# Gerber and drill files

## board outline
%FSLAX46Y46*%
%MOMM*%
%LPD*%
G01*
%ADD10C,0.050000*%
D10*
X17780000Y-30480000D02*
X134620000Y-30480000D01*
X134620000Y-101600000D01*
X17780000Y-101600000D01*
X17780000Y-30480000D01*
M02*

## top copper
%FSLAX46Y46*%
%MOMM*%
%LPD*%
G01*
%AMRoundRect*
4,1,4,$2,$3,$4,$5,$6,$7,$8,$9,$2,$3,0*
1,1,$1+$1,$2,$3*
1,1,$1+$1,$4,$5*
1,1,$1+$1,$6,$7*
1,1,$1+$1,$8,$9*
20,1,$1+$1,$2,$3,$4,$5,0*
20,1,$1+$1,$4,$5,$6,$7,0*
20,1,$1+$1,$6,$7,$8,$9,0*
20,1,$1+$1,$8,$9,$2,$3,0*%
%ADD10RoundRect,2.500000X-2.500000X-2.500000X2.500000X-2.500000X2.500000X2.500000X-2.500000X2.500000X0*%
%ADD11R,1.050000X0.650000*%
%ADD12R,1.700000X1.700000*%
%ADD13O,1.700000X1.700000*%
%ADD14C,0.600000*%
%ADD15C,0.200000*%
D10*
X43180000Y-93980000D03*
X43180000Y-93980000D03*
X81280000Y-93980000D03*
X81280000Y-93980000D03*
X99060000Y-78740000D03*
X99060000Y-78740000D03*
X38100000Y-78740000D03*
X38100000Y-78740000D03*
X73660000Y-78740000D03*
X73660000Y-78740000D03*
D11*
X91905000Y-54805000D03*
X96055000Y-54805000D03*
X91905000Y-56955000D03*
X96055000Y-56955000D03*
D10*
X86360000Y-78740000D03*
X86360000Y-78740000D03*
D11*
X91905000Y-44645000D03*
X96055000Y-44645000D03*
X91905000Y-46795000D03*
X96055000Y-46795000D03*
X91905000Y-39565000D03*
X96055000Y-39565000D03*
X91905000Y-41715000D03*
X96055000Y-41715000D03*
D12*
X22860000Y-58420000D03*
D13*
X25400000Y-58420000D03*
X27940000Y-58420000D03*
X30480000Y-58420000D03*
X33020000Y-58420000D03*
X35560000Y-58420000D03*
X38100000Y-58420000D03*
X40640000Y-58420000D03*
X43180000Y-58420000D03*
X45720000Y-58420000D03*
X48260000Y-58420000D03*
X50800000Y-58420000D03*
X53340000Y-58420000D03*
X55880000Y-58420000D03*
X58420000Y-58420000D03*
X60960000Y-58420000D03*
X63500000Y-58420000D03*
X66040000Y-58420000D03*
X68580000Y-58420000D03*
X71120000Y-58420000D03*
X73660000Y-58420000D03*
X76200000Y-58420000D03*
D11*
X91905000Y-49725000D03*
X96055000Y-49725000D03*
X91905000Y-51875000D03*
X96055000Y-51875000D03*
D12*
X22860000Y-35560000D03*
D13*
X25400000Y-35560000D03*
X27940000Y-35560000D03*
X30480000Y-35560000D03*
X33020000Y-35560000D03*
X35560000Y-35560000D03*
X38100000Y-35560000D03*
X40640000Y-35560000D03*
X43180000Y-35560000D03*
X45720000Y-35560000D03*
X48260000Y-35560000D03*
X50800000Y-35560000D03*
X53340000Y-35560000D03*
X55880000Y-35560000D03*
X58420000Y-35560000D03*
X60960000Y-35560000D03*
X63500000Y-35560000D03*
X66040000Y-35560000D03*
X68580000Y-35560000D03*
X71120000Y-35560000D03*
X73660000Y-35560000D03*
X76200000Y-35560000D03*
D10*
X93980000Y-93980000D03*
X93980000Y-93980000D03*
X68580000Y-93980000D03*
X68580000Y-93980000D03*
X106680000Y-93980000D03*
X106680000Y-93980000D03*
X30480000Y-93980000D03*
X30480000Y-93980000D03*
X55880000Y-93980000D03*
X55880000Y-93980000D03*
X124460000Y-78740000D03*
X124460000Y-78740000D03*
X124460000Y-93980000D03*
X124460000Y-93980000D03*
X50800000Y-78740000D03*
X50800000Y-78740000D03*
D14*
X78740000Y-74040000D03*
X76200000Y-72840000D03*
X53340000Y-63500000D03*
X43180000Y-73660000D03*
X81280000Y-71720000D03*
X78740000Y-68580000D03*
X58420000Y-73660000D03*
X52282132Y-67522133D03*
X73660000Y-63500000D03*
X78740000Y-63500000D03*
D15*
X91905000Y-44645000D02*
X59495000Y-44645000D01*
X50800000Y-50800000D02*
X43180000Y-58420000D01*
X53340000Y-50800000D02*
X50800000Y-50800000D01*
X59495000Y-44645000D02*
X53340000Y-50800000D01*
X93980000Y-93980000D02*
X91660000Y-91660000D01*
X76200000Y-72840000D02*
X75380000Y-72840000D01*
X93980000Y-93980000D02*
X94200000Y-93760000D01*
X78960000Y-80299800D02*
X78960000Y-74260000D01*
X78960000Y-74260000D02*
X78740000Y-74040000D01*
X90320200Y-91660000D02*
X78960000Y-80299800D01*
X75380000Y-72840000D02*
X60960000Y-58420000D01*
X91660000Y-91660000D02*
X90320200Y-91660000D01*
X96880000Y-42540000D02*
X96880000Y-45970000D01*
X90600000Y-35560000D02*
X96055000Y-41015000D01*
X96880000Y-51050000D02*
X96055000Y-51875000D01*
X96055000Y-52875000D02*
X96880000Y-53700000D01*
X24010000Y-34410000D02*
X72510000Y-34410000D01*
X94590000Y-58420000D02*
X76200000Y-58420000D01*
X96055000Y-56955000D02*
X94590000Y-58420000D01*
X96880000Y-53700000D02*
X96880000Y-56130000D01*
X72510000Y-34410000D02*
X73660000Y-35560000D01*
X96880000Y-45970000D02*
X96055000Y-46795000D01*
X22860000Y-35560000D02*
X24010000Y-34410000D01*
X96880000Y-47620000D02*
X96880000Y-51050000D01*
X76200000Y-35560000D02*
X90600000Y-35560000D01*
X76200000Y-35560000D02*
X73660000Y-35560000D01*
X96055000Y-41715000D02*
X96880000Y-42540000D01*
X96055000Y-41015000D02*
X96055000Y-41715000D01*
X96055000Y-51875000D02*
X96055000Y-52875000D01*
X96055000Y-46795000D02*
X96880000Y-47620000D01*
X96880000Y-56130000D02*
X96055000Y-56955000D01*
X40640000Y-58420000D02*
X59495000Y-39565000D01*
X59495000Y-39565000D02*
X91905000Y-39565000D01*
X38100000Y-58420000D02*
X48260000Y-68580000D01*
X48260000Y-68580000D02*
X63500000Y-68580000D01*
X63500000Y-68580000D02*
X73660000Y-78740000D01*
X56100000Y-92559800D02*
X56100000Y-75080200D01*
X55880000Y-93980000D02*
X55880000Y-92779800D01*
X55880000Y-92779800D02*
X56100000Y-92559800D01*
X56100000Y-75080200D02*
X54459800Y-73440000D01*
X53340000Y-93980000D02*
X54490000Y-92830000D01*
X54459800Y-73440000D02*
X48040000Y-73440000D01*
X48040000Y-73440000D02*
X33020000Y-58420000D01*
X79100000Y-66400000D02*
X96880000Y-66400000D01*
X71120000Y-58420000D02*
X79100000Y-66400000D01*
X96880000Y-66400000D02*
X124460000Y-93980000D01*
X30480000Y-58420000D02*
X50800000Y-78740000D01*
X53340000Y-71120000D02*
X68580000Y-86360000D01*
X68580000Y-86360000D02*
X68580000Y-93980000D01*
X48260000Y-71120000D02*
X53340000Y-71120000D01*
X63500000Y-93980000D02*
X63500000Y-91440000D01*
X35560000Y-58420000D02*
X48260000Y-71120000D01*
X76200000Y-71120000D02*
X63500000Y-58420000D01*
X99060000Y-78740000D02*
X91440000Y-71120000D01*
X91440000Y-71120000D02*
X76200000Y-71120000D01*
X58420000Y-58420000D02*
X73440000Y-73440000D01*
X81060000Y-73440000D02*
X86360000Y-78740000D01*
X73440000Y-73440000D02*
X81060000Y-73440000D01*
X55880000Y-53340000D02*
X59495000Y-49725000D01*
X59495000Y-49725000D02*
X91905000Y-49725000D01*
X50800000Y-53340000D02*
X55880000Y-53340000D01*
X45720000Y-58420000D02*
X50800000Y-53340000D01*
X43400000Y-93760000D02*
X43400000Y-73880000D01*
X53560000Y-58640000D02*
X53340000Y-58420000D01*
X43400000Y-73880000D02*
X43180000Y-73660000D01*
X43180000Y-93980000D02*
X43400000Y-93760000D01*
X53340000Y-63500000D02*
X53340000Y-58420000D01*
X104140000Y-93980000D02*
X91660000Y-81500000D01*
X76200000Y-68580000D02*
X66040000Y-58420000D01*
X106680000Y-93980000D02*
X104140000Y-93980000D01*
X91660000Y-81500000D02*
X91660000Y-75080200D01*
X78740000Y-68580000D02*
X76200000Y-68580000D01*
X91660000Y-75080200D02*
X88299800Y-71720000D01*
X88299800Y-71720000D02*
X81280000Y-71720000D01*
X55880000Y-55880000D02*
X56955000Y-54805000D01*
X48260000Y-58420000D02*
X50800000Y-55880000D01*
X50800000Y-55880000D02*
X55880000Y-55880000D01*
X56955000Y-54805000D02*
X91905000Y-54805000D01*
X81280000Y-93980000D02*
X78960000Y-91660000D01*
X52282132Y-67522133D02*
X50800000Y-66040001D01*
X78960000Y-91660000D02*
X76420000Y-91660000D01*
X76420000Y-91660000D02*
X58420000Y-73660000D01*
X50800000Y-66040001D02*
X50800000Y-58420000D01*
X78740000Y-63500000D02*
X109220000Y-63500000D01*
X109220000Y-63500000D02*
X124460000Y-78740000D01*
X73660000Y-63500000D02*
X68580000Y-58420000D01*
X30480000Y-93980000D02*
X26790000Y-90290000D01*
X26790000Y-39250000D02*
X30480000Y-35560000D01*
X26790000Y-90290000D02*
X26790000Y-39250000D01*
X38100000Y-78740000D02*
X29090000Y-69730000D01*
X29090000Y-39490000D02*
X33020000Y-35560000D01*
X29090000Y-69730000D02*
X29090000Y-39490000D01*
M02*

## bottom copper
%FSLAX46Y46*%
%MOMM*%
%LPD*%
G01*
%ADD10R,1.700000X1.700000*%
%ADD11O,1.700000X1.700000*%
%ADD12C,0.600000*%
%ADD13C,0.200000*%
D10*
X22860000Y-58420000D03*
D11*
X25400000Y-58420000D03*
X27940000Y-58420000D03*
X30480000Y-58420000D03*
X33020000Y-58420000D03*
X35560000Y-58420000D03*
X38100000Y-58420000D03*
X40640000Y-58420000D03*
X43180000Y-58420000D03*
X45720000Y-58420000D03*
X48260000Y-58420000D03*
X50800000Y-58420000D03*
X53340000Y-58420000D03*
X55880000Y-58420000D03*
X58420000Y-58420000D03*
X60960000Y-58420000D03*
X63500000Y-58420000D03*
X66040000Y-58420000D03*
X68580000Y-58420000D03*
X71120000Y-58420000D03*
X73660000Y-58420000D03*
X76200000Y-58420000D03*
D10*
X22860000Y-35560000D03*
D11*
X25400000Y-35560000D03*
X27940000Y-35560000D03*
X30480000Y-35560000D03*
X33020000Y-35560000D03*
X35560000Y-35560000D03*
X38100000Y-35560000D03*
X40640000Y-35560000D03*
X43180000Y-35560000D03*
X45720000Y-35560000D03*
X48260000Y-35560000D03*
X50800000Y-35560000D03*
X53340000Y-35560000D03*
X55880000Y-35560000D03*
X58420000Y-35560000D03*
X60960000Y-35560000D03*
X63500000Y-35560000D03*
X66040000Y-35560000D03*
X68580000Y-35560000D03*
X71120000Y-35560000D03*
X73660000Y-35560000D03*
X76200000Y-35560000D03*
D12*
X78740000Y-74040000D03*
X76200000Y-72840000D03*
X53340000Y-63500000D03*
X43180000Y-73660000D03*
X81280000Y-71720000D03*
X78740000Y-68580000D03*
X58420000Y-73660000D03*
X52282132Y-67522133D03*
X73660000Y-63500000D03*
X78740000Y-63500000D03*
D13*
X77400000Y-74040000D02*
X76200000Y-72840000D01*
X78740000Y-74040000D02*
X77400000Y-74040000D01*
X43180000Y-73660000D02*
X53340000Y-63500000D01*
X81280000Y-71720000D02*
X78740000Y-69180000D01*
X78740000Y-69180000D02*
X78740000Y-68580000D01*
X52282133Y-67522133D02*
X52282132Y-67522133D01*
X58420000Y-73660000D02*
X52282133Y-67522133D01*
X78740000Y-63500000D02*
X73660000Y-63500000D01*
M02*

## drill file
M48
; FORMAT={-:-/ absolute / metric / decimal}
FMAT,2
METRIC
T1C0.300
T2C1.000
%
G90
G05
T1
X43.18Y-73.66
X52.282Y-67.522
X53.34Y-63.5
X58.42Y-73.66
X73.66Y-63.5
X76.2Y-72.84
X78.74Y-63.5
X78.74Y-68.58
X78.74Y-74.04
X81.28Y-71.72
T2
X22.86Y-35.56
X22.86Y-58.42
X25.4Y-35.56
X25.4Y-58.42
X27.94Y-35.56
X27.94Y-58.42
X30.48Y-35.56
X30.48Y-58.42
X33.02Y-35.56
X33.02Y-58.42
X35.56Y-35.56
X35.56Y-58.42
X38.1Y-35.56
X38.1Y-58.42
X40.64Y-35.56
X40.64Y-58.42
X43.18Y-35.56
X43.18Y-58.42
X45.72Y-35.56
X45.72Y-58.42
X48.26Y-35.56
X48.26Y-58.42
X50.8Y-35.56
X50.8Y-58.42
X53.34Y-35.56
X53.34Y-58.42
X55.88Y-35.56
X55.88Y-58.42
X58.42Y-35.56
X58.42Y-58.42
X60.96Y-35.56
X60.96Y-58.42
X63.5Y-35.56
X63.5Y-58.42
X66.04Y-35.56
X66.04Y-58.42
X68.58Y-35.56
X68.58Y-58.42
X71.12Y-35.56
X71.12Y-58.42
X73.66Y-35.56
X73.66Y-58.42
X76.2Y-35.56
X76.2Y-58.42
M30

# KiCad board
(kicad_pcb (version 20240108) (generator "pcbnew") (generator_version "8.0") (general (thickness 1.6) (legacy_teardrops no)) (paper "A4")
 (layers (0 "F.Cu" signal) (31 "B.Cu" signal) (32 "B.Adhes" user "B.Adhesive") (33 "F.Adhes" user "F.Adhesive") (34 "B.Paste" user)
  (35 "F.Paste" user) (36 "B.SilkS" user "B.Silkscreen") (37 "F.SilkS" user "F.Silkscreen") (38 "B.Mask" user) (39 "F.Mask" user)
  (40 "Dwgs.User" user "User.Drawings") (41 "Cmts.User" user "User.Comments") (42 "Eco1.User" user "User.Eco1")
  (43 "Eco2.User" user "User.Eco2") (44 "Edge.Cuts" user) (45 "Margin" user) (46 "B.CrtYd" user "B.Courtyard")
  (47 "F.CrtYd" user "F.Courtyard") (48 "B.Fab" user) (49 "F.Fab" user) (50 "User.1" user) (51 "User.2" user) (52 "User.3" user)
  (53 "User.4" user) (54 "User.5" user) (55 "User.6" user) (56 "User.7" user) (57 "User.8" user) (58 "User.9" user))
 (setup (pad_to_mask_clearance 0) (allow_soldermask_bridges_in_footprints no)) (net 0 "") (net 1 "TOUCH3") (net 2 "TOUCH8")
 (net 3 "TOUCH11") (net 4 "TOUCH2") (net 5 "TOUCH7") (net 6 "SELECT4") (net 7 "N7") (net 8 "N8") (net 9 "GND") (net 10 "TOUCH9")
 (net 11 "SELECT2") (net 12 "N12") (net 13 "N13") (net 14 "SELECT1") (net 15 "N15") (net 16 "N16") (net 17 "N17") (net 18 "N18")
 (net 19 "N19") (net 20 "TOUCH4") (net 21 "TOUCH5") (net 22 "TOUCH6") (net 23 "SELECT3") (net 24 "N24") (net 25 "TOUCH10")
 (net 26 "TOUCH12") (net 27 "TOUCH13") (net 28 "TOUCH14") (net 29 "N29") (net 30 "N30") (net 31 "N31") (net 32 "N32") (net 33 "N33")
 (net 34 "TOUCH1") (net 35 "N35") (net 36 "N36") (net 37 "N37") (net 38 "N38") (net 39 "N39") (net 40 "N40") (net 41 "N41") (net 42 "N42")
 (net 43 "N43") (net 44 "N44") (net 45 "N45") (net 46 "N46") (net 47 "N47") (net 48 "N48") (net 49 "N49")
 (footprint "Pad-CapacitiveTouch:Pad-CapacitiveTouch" (layer "F.Cu") (at 43.18 93.98)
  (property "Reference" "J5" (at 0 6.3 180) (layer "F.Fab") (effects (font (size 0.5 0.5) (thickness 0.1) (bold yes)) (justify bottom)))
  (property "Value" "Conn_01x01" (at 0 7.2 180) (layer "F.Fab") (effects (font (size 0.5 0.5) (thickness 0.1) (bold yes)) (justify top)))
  (pad "1" smd roundrect (at 0 0) (size 10 10) (layers "F.Cu") (roundrect_rratio 0.25) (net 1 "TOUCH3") (thermal_bridge_angle 0))
  (pad "1" smd roundrect (at 0 0) (size 10 10) (layers "F.Cu" "F.Mask") (roundrect_rratio 0.25) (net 1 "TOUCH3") (thermal_bridge_angle 0)))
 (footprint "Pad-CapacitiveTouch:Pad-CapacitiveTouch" (layer "F.Cu") (at 81.28 93.98)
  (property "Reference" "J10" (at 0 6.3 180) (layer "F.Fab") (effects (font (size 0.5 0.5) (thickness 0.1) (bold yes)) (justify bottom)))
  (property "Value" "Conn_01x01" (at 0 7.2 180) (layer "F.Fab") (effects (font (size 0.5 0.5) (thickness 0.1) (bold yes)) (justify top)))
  (pad "1" smd roundrect (at 0 0) (size 10 10) (layers "F.Cu") (roundrect_rratio 0.25) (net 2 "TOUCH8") (thermal_bridge_angle 0))
  (pad "1" smd roundrect (at 0 0) (size 10 10) (layers "F.Cu" "F.Mask") (roundrect_rratio 0.25) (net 2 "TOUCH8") (thermal_bridge_angle 0)))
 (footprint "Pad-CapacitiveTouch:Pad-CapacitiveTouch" (layer "F.Cu") (at 99.06 78.74)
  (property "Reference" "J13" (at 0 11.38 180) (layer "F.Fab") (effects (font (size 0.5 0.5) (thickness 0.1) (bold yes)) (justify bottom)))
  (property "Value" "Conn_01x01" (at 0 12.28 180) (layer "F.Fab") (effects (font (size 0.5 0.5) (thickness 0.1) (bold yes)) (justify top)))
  (pad "1" smd roundrect (at 0 0) (size 10 10) (layers "F.Cu") (roundrect_rratio 0.25) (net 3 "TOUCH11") (thermal_bridge_angle 0))
  (pad "1" smd roundrect (at 0 0) (size 10 10) (layers "F.Cu" "F.Mask") (roundrect_rratio 0.25) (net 3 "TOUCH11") (thermal_bridge_angle 0)))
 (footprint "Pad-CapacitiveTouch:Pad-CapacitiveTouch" (layer "F.Cu") (at 38.1 78.74)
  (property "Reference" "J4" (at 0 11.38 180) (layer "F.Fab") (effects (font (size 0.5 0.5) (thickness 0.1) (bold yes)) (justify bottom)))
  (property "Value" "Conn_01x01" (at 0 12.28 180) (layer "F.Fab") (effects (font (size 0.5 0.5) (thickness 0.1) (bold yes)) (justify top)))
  (pad "1" smd roundrect (at 0 0) (size 10 10) (layers "F.Cu") (roundrect_rratio 0.25) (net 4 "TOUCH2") (thermal_bridge_angle 0))
  (pad "1" smd roundrect (at 0 0) (size 10 10) (layers "F.Cu" "F.Mask") (roundrect_rratio 0.25) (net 4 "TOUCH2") (thermal_bridge_angle 0)))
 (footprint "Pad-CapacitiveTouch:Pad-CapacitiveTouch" (layer "F.Cu") (at 73.66 78.74)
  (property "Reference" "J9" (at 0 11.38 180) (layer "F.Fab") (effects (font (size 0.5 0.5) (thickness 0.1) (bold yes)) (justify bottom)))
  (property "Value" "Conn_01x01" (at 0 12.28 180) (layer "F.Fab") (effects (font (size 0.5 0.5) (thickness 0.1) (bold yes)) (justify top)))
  (pad "1" smd roundrect (at 0 0) (size 10 10) (layers "F.Cu") (roundrect_rratio 0.25) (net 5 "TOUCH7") (thermal_bridge_angle 0))
  (pad "1" smd roundrect (at 0 0) (size 10 10) (layers "F.Cu" "F.Mask") (roundrect_rratio 0.25) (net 5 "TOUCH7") (thermal_bridge_angle 0)))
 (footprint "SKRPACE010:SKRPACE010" (layer "F.Cu") (at 93.98 55.88)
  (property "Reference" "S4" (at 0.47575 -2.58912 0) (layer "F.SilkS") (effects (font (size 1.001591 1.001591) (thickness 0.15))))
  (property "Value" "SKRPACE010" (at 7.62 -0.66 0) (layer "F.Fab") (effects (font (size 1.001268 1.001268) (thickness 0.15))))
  (pad "1" smd rect (at -2.075 -1.075) (size 1.05 0.65) (layers "F.Cu" "F.Paste" "F.Mask") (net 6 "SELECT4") (solder_mask_margin 0.102))
  (pad "2" smd rect (at 2.075 -1.075) (size 1.05 0.65) (layers "F.Cu" "F.Paste" "F.Mask") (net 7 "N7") (solder_mask_margin 0.102))
  (pad "3" smd rect (at -2.075 1.075) (size 1.05 0.65) (layers "F.Cu" "F.Paste" "F.Mask") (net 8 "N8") (solder_mask_margin 0.102))
  (pad "4" smd rect (at 2.075 1.075) (size 1.05 0.65) (layers "F.Cu" "F.Paste" "F.Mask") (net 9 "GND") (solder_mask_margin 0.102)))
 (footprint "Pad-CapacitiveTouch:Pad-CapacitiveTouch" (layer "F.Cu") (at 86.36 78.74)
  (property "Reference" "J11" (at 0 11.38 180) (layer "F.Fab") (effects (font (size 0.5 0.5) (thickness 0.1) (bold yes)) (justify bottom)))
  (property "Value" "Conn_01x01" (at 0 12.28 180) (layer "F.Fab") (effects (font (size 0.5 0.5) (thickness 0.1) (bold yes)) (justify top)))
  (pad "1" smd roundrect (at 0 0) (size 10 10) (layers "F.Cu") (roundrect_rratio 0.25) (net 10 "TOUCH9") (thermal_bridge_angle 0))
  (pad "1" smd roundrect (at 0 0) (size 10 10) (layers "F.Cu" "F.Mask") (roundrect_rratio 0.25) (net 10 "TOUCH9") (thermal_bridge_angle 0)))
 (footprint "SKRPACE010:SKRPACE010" (layer "F.Cu") (at 93.98 45.72)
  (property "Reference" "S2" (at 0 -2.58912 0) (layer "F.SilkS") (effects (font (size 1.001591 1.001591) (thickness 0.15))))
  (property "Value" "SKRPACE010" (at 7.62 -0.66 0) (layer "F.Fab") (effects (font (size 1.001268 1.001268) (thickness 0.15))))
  (pad "1" smd rect (at -2.075 -1.075) (size 1.05 0.65) (layers "F.Cu" "F.Paste" "F.Mask") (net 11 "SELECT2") (solder_mask_margin 0.102))
  (pad "2" smd rect (at 2.075 -1.075) (size 1.05 0.65) (layers "F.Cu" "F.Paste" "F.Mask") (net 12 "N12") (solder_mask_margin 0.102))
  (pad "3" smd rect (at -2.075 1.075) (size 1.05 0.65) (layers "F.Cu" "F.Paste" "F.Mask") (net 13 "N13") (solder_mask_margin 0.102))
  (pad "4" smd rect (at 2.075 1.075) (size 1.05 0.65) (layers "F.Cu" "F.Paste" "F.Mask") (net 9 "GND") (solder_mask_margin 0.102)))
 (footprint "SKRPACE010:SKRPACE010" (layer "F.Cu") (at 93.98 40.64)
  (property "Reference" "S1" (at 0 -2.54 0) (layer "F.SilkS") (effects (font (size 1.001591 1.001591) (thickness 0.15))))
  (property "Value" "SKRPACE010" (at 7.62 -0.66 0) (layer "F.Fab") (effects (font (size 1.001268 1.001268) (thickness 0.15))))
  (pad "1" smd rect (at -2.075 -1.075) (size 1.05 0.65) (layers "F.Cu" "F.Paste" "F.Mask") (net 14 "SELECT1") (solder_mask_margin 0.102))
  (pad "2" smd rect (at 2.075 -1.075) (size 1.05 0.65) (layers "F.Cu" "F.Paste" "F.Mask") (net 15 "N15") (solder_mask_margin 0.102))
  (pad "3" smd rect (at -2.075 1.075) (size 1.05 0.65) (layers "F.Cu" "F.Paste" "F.Mask") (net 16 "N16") (solder_mask_margin 0.102))
  (pad "4" smd rect (at 2.075 1.075) (size 1.05 0.65) (layers "F.Cu" "F.Paste" "F.Mask") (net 9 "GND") (solder_mask_margin 0.102)))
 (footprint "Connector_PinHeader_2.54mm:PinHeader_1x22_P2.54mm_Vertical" (layer "F.Cu") (at 22.86 58.42 90)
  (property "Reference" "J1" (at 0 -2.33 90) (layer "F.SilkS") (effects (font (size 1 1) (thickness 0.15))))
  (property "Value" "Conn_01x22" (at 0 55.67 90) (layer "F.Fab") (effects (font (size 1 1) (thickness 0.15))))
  (pad "1" thru_hole rect (at 0 0 90) (size 1.7 1.7) (drill 1) (layers "*.Cu" "*.Mask") (remove_unused_layers no) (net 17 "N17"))
  (pad "2" thru_hole oval (at 0 2.54 90) (size 1.7 1.7) (drill 1) (layers "*.Cu" "*.Mask") (remove_unused_layers no) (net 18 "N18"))
  (pad "3" thru_hole oval (at 0 5.08 90) (size 1.7 1.7) (drill 1) (layers "*.Cu" "*.Mask") (remove_unused_layers no) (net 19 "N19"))
  (pad "4" thru_hole oval (at 0 7.62 90) (size 1.7 1.7) (drill 1) (layers "*.Cu" "*.Mask") (remove_unused_layers no) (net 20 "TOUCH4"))
  (pad "5" thru_hole oval (at 0 10.16 90) (size 1.7 1.7) (drill 1) (layers "*.Cu" "*.Mask") (remove_unused_layers no) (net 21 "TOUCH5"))
  (pad "6" thru_hole oval (at 0 12.7 90) (size 1.7 1.7) (drill 1) (layers "*.Cu" "*.Mask") (remove_unused_layers no) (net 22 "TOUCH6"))
  (pad "7" thru_hole oval (at 0 15.24 90) (size 1.7 1.7) (drill 1) (layers "*.Cu" "*.Mask") (remove_unused_layers no) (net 5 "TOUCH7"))
  (pad "8" thru_hole oval (at 0 17.78 90) (size 1.7 1.7) (drill 1) (layers "*.Cu" "*.Mask") (remove_unused_layers no) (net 14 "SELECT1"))
  (pad "9" thru_hole oval (at 0 20.32 90) (size 1.7 1.7) (drill 1) (layers "*.Cu" "*.Mask") (remove_unused_layers no) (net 11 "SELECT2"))
  (pad "10" thru_hole oval (at 0 22.86 90) (size 1.7 1.7) (drill 1) (layers "*.Cu" "*.Mask") (remove_unused_layers no) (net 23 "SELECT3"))
  (pad "11" thru_hole oval (at 0 25.4 90) (size 1.7 1.7) (drill 1) (layers "*.Cu" "*.Mask") (remove_unused_layers no) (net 6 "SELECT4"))
  (pad "12" thru_hole oval (at 0 27.94 90) (size 1.7 1.7) (drill 1) (layers "*.Cu" "*.Mask") (remove_unused_layers no) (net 2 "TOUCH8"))
  (pad "13" thru_hole oval (at 0 30.48 90) (size 1.7 1.7) (drill 1) (layers "*.Cu" "*.Mask") (remove_unused_layers no) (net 1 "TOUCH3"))
  (pad "14" thru_hole oval (at 0 33.02 90) (size 1.7 1.7) (drill 1) (layers "*.Cu" "*.Mask") (remove_unused_layers no) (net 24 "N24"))
  (pad "15" thru_hole oval (at 0 35.56 90) (size 1.7 1.7) (drill 1) (layers "*.Cu" "*.Mask") (remove_unused_layers no) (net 10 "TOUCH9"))
  (pad "16" thru_hole oval (at 0 38.1 90) (size 1.7 1.7) (drill 1) (layers "*.Cu" "*.Mask") (remove_unused_layers no) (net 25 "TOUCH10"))
  (pad "17" thru_hole oval (at 0 40.64 90) (size 1.7 1.7) (drill 1) (layers "*.Cu" "*.Mask") (remove_unused_layers no) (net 3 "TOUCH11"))
  (pad "18" thru_hole oval (at 0 43.18 90) (size 1.7 1.7) (drill 1) (layers "*.Cu" "*.Mask") (remove_unused_layers no) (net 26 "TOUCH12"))
  (pad "19" thru_hole oval (at 0 45.72 90) (size 1.7 1.7) (drill 1) (layers "*.Cu" "*.Mask") (remove_unused_layers no) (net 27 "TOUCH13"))
  (pad "20" thru_hole oval (at 0 48.26 90) (size 1.7 1.7) (drill 1) (layers "*.Cu" "*.Mask") (remove_unused_layers no) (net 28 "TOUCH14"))
  (pad "21" thru_hole oval (at 0 50.8 90) (size 1.7 1.7) (drill 1) (layers "*.Cu" "*.Mask") (remove_unused_layers no) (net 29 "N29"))
  (pad "22" thru_hole oval (at 0 53.34 90) (size 1.7 1.7) (drill 1) (layers "*.Cu" "*.Mask") (remove_unused_layers no) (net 9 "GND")))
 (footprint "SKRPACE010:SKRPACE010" (layer "F.Cu") (at 93.98 50.8)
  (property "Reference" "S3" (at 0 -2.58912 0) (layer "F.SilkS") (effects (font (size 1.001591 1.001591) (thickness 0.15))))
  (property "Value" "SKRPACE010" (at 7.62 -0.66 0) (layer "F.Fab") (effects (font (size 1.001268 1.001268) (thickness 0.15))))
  (pad "1" smd rect (at -2.075 -1.075) (size 1.05 0.65) (layers "F.Cu" "F.Paste" "F.Mask") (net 23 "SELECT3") (solder_mask_margin 0.102))
  (pad "2" smd rect (at 2.075 -1.075) (size 1.05 0.65) (layers "F.Cu" "F.Paste" "F.Mask") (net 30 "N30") (solder_mask_margin 0.102))
  (pad "3" smd rect (at -2.075 1.075) (size 1.05 0.65) (layers "F.Cu" "F.Paste" "F.Mask") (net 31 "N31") (solder_mask_margin 0.102))
  (pad "4" smd rect (at 2.075 1.075) (size 1.05 0.65) (layers "F.Cu" "F.Paste" "F.Mask") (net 9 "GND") (solder_mask_margin 0.102)))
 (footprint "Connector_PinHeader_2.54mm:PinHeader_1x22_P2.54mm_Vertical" (layer "F.Cu") (at 22.86 35.56 90)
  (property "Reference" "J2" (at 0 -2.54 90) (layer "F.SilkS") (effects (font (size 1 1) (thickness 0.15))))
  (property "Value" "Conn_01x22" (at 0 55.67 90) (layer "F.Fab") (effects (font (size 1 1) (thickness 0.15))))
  (pad "1" thru_hole rect (at 0 0 90) (size 1.7 1.7) (drill 1) (layers "*.Cu" "*.Mask") (remove_unused_layers no) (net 9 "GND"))
  (pad "2" thru_hole oval (at 0 2.54 90) (size 1.7 1.7) (drill 1) (layers "*.Cu" "*.Mask") (remove_unused_layers no) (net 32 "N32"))
  (pad "3" thru_hole oval (at 0 5.08 90) (size 1.7 1.7) (drill 1) (layers "*.Cu" "*.Mask") (remove_unused_layers no) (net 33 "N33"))
  (pad "4" thru_hole oval (at 0 7.62 90) (size 1.7 1.7) (drill 1) (layers "*.Cu" "*.Mask") (remove_unused_layers no) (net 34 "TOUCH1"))
  (pad "5" thru_hole oval (at 0 10.16 90) (size 1.7 1.7) (drill 1) (layers "*.Cu" "*.Mask") (remove_unused_layers no) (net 4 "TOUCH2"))
  (pad "6" thru_hole oval (at 0 12.7 90) (size 1.7 1.7) (drill 1) (layers "*.Cu" "*.Mask") (remove_unused_layers no) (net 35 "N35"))
  (pad "7" thru_hole oval (at 0 15.24 90) (size 1.7 1.7) (drill 1) (layers "*.Cu" "*.Mask") (remove_unused_layers no) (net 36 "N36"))
  (pad "8" thru_hole oval (at 0 17.78 90) (size 1.7 1.7) (drill 1) (layers "*.Cu" "*.Mask") (remove_unused_layers no) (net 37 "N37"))
  (pad "9" thru_hole oval (at 0 20.32 90) (size 1.7 1.7) (drill 1) (layers "*.Cu" "*.Mask") (remove_unused_layers no) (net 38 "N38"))
  (pad "10" thru_hole oval (at 0 22.86 90) (size 1.7 1.7) (drill 1) (layers "*.Cu" "*.Mask") (remove_unused_layers no) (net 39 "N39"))
  (pad "11" thru_hole oval (at 0 25.4 90) (size 1.7 1.7) (drill 1) (layers "*.Cu" "*.Mask") (remove_unused_layers no) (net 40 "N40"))
  (pad "12" thru_hole oval (at 0 27.94 90) (size 1.7 1.7) (drill 1) (layers "*.Cu" "*.Mask") (remove_unused_layers no) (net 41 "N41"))
  (pad "13" thru_hole oval (at 0 30.48 90) (size 1.7 1.7) (drill 1) (layers "*.Cu" "*.Mask") (remove_unused_layers no) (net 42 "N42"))
  (pad "14" thru_hole oval (at 0 33.02 90) (size 1.7 1.7) (drill 1) (layers "*.Cu" "*.Mask") (remove_unused_layers no) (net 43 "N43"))
  (pad "15" thru_hole oval (at 0 35.56 90) (size 1.7 1.7) (drill 1) (layers "*.Cu" "*.Mask") (remove_unused_layers no) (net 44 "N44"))
  (pad "16" thru_hole oval (at 0 38.1 90) (size 1.7 1.7) (drill 1) (layers "*.Cu" "*.Mask") (remove_unused_layers no) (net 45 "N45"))
  (pad "17" thru_hole oval (at 0 40.64 90) (size 1.7 1.7) (drill 1) (layers "*.Cu" "*.Mask") (remove_unused_layers no) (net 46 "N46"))
  (pad "18" thru_hole oval (at 0 43.18 90) (size 1.7 1.7) (drill 1) (layers "*.Cu" "*.Mask") (remove_unused_layers no) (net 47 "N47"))
  (pad "19" thru_hole oval (at 0 45.72 90) (size 1.7 1.7) (drill 1) (layers "*.Cu" "*.Mask") (remove_unused_layers no) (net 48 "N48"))
  (pad "20" thru_hole oval (at 0 48.26 90) (size 1.7 1.7) (drill 1) (layers "*.Cu" "*.Mask") (remove_unused_layers no) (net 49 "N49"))
  (pad "21" thru_hole oval (at 0 50.8 90) (size 1.7 1.7) (drill 1) (layers "*.Cu" "*.Mask") (remove_unused_layers no) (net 9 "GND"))
  (pad "22" thru_hole oval (at 0 53.34 90) (size 1.7 1.7) (drill 1) (layers "*.Cu" "*.Mask") (remove_unused_layers no) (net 9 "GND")))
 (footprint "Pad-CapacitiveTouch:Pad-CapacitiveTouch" (layer "F.Cu") (at 93.98 93.98)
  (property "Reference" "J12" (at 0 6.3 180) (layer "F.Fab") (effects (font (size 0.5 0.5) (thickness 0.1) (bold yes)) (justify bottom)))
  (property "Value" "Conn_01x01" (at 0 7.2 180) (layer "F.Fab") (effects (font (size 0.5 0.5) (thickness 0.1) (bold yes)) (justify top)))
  (pad "1" smd roundrect (at 0 0) (size 10 10) (layers "F.Cu") (roundrect_rratio 0.25) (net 25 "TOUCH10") (thermal_bridge_angle 0))
  (pad "1" smd roundrect (at 0 0) (size 10 10) (layers "F.Cu" "F.Mask") (roundrect_rratio 0.25) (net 25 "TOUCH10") (thermal_bridge_angle 0)))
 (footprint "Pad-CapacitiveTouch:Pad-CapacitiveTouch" (layer "F.Cu") (at 68.58 93.98)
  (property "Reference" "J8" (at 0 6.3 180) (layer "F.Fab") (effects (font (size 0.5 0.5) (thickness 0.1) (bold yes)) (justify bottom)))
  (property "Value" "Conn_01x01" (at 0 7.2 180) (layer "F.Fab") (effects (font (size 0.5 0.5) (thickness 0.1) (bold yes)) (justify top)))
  (pad "1" smd roundrect (at 0 0) (size 10 10) (layers "F.Cu") (roundrect_rratio 0.25) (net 22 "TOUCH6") (thermal_bridge_angle 0))
  (pad "1" smd roundrect (at 0 0) (size 10 10) (layers "F.Cu" "F.Mask") (roundrect_rratio 0.25) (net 22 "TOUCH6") (thermal_bridge_angle 0)))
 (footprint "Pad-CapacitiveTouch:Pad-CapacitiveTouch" (layer "F.Cu") (at 106.68 93.98)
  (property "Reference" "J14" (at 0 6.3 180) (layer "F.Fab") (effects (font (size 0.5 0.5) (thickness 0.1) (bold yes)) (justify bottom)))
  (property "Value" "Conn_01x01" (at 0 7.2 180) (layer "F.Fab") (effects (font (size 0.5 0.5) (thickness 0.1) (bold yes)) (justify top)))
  (pad "1" smd roundrect (at 0 0) (size 10 10) (layers "F.Cu") (roundrect_rratio 0.25) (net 26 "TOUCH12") (thermal_bridge_angle 0))
  (pad "1" smd roundrect (at 0 0) (size 10 10) (layers "F.Cu" "F.Mask") (roundrect_rratio 0.25) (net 26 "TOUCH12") (thermal_bridge_angle 0)))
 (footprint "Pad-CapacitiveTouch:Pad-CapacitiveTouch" (layer "F.Cu") (at 30.48 93.98)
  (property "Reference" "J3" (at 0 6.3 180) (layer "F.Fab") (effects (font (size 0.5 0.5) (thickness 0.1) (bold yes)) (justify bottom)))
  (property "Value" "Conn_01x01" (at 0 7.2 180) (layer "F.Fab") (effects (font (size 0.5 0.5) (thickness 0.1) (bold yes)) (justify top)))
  (pad "1" smd roundrect (at 0 0) (size 10 10) (layers "F.Cu") (roundrect_rratio 0.25) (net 34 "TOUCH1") (thermal_bridge_angle 0))
  (pad "1" smd roundrect (at 0 0) (size 10 10) (layers "F.Cu" "F.Mask") (roundrect_rratio 0.25) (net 34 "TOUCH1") (thermal_bridge_angle 0)))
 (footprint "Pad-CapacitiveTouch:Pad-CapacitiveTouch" (layer "F.Cu") (at 55.88 93.98)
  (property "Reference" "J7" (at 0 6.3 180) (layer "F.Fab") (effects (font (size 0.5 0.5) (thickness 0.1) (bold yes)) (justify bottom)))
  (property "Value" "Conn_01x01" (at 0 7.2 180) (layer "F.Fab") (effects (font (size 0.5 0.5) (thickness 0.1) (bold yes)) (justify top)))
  (pad "1" smd roundrect (at 0 0) (size 10 10) (layers "F.Cu") (roundrect_rratio 0.25) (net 21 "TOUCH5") (thermal_bridge_angle 0))
  (pad "1" smd roundrect (at 0 0) (size 10 10) (layers "F.Cu" "F.Mask") (roundrect_rratio 0.25) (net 21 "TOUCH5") (thermal_bridge_angle 0)))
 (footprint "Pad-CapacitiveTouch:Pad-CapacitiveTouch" (layer "F.Cu") (at 124.46 78.74)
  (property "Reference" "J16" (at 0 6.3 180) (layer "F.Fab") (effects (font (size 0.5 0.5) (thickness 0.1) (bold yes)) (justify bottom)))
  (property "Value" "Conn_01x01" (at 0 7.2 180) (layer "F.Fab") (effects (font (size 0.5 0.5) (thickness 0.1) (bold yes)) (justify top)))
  (pad "1" smd roundrect (at 0 0) (size 10 10) (layers "F.Cu") (roundrect_rratio 0.25) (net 27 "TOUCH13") (thermal_bridge_angle 0))
  (pad "1" smd roundrect (at 0 0) (size 10 10) (layers "F.Cu" "F.Mask") (roundrect_rratio 0.25) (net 27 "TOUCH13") (thermal_bridge_angle 0)))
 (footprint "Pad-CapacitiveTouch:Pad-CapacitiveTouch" (layer "F.Cu") (at 124.46 93.98)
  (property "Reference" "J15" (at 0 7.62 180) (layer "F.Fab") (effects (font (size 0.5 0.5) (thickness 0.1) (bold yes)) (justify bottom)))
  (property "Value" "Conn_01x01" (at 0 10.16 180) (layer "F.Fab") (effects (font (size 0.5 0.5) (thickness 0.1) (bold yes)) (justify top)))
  (pad "1" smd roundrect (at 0 0) (size 10 10) (layers "F.Cu") (roundrect_rratio 0.25) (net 28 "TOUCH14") (thermal_bridge_angle 0))
  (pad "1" smd roundrect (at 0 0) (size 10 10) (layers "F.Cu" "F.Mask") (roundrect_rratio 0.25) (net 28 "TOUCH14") (thermal_bridge_angle 0)))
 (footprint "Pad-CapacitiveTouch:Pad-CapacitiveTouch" (layer "F.Cu") (at 50.8 78.74)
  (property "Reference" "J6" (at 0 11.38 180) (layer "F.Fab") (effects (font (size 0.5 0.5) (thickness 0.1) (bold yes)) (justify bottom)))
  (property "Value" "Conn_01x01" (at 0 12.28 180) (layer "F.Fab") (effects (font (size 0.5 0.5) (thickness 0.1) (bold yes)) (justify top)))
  (pad "1" smd roundrect (at 0 0) (size 10 10) (layers "F.Cu") (roundrect_rratio 0.25) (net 20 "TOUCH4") (thermal_bridge_angle 0))
  (pad "1" smd roundrect (at 0 0) (size 10 10) (layers "F.Cu" "F.Mask") (roundrect_rratio 0.25) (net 20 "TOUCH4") (thermal_bridge_angle 0)))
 (gr_rect (start 17.78 30.48) (end 134.62 101.6) (stroke (width 0.05) (type default)) (fill none) (layer "Edge.Cuts"))
 (segment (start 91.905 44.645) (end 59.495 44.645) (width 0.2) (layer "F.Cu") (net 11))
 (segment (start 50.8 50.8) (end 43.18 58.42) (width 0.2) (layer "F.Cu") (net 11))
 (segment (start 53.34 50.8) (end 50.8 50.8) (width 0.2) (layer "F.Cu") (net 11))
 (segment (start 59.495 44.645) (end 53.34 50.8) (width 0.2) (layer "F.Cu") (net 11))
 (segment (start 93.98 93.98) (end 91.66 91.66) (width 0.2) (layer "F.Cu") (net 25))
 (segment (start 76.2 72.84) (end 75.38 72.84) (width 0.2) (layer "F.Cu") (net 25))
 (segment (start 93.98 93.98) (end 94.2 93.76) (width 0.2) (layer "F.Cu") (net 25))
 (segment (start 78.96 80.2998) (end 78.96 74.26) (width 0.2) (layer "F.Cu") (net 25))
 (segment (start 78.96 74.26) (end 78.74 74.04) (width 0.2) (layer "F.Cu") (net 25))
 (segment (start 90.3202 91.66) (end 78.96 80.2998) (width 0.2) (layer "F.Cu") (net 25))
 (segment (start 75.38 72.84) (end 60.96 58.42) (width 0.2) (layer "F.Cu") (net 25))
 (segment (start 91.66 91.66) (end 90.3202 91.66) (width 0.2) (layer "F.Cu") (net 25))
 (via (at 78.74 74.04) (size 0.6) (drill 0.3) (layers "F.Cu" "B.Cu") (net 25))
 (via (at 76.2 72.84) (size 0.6) (drill 0.3) (layers "F.Cu" "B.Cu") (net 25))
 (segment (start 77.4 74.04) (end 76.2 72.84) (width 0.2) (layer "B.Cu") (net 25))
 (segment (start 78.74 74.04) (end 77.4 74.04) (width 0.2) (layer "B.Cu") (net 25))
 (segment (start 96.88 42.54) (end 96.88 45.97) (width 0.2) (layer "F.Cu") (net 9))
 (segment (start 90.6 35.56) (end 96.055 41.015) (width 0.2) (layer "F.Cu") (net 9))
 (segment (start 96.88 51.05) (end 96.055 51.875) (width 0.2) (layer "F.Cu") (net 9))
 (segment (start 96.055 52.875) (end 96.88 53.7) (width 0.2) (layer "F.Cu") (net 9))
 (segment (start 24.01 34.41) (end 72.51 34.41) (width 0.2) (layer "F.Cu") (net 9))
 (segment (start 94.59 58.42) (end 76.2 58.42) (width 0.2) (layer "F.Cu") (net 9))
 (segment (start 96.055 56.955) (end 94.59 58.42) (width 0.2) (layer "F.Cu") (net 9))
 (segment (start 96.88 53.7) (end 96.88 56.13) (width 0.2) (layer "F.Cu") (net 9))
 (segment (start 72.51 34.41) (end 73.66 35.56) (width 0.2) (layer "F.Cu") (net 9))
 (segment (start 96.88 45.97) (end 96.055 46.795) (width 0.2) (layer "F.Cu") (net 9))
 (segment (start 22.86 35.56) (end 24.01 34.41) (width 0.2) (layer "F.Cu") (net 9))
 (segment (start 96.88 47.62) (end 96.88 51.05) (width 0.2) (layer "F.Cu") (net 9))
 (segment (start 76.2 35.56) (end 90.6 35.56) (width 0.2) (layer "F.Cu") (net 9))
 (segment (start 76.2 35.56) (end 73.66 35.56) (width 0.2) (layer "F.Cu") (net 9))
 (segment (start 96.055 41.715) (end 96.88 42.54) (width 0.2) (layer "F.Cu") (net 9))
 (segment (start 96.055 41.015) (end 96.055 41.715) (width 0.2) (layer "F.Cu") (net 9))
 (segment (start 96.055 51.875) (end 96.055 52.875) (width 0.2) (layer "F.Cu") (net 9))
 (segment (start 96.055 46.795) (end 96.88 47.62) (width 0.2) (layer "F.Cu") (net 9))
 (segment (start 96.88 56.13) (end 96.055 56.955) (width 0.2) (layer "F.Cu") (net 9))
 (segment (start 40.64 58.42) (end 59.495 39.565) (width 0.2) (layer "F.Cu") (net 14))
 (segment (start 59.495 39.565) (end 91.905 39.565) (width 0.2) (layer "F.Cu") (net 14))
 (segment (start 38.1 58.42) (end 48.26 68.58) (width 0.2) (layer "F.Cu") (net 5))
 (segment (start 48.26 68.58) (end 63.5 68.58) (width 0.2) (layer "F.Cu") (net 5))
 (segment (start 63.5 68.58) (end 73.66 78.74) (width 0.2) (layer "F.Cu") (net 5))
 (segment (start 56.1 92.5598) (end 56.1 75.0802) (width 0.2) (layer "F.Cu") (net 21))
 (segment (start 55.88 93.98) (end 55.88 92.7798) (width 0.2) (layer "F.Cu") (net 21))
 (segment (start 55.88 92.7798) (end 56.1 92.5598) (width 0.2) (layer "F.Cu") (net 21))
 (segment (start 56.1 75.0802) (end 54.4598 73.44) (width 0.2) (layer "F.Cu") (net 21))
 (segment (start 53.34 93.98) (end 54.49 92.83) (width 0.2) (layer "F.Cu") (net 21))
 (segment (start 54.4598 73.44) (end 48.04 73.44) (width 0.2) (layer "F.Cu") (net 21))
 (segment (start 48.04 73.44) (end 33.02 58.42) (width 0.2) (layer "F.Cu") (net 21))
 (segment (start 79.1 66.4) (end 96.88 66.4) (width 0.2) (layer "F.Cu") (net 28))
 (segment (start 71.12 58.42) (end 79.1 66.4) (width 0.2) (layer "F.Cu") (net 28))
 (segment (start 96.88 66.4) (end 124.46 93.98) (width 0.2) (layer "F.Cu") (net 28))
 (segment (start 30.48 58.42) (end 50.8 78.74) (width 0.2) (layer "F.Cu") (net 20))
 (segment (start 53.34 71.12) (end 68.58 86.36) (width 0.2) (layer "F.Cu") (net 22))
 (segment (start 68.58 86.36) (end 68.58 93.98) (width 0.2) (layer "F.Cu") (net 22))
 (segment (start 48.26 71.12) (end 53.34 71.12) (width 0.2) (layer "F.Cu") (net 22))
 (segment (start 63.5 93.98) (end 63.5 91.44) (width 0.2) (layer "F.Cu") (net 22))
 (segment (start 35.56 58.42) (end 48.26 71.12) (width 0.2) (layer "F.Cu") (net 22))
 (segment (start 76.2 71.12) (end 63.5 58.42) (width 0.2) (layer "F.Cu") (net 3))
 (segment (start 99.06 78.74) (end 91.44 71.12) (width 0.2) (layer "F.Cu") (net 3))
 (segment (start 91.44 71.12) (end 76.2 71.12) (width 0.2) (layer "F.Cu") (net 3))
 (segment (start 58.42 58.42) (end 73.44 73.44) (width 0.2) (layer "F.Cu") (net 10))
 (segment (start 81.06 73.44) (end 86.36 78.74) (width 0.2) (layer "F.Cu") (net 10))
 (segment (start 73.44 73.44) (end 81.06 73.44) (width 0.2) (layer "F.Cu") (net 10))
 (segment (start 55.88 53.34) (end 59.495 49.725) (width 0.2) (layer "F.Cu") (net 23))
 (segment (start 59.495 49.725) (end 91.905 49.725) (width 0.2) (layer "F.Cu") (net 23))
 (segment (start 50.8 53.34) (end 55.88 53.34) (width 0.2) (layer "F.Cu") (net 23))
 (segment (start 45.72 58.42) (end 50.8 53.34) (width 0.2) (layer "F.Cu") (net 23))
 (segment (start 43.4 93.76) (end 43.4 73.88) (width 0.2) (layer "F.Cu") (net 1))
 (segment (start 53.56 58.64) (end 53.34 58.42) (width 0.2) (layer "F.Cu") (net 1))
 (segment (start 43.4 73.88) (end 43.18 73.66) (width 0.2) (layer "F.Cu") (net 1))
 (segment (start 43.18 93.98) (end 43.4 93.76) (width 0.2) (layer "F.Cu") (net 1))
 (segment (start 53.34 63.5) (end 53.34 58.42) (width 0.2) (layer "F.Cu") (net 1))
 (via (at 53.34 63.5) (size 0.6) (drill 0.3) (layers "F.Cu" "B.Cu") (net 1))
 (via (at 43.18 73.66) (size 0.6) (drill 0.3) (layers "F.Cu" "B.Cu") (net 1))
 (segment (start 43.18 73.66) (end 53.34 63.5) (width 0.2) (layer "B.Cu") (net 1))
 (segment (start 104.14 93.98) (end 91.66 81.5) (width 0.2) (layer "F.Cu") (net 26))
 (segment (start 76.2 68.58) (end 66.04 58.42) (width 0.2) (layer "F.Cu") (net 26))
 (segment (start 106.68 93.98) (end 104.14 93.98) (width 0.2) (layer "F.Cu") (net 26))
 (segment (start 91.66 81.5) (end 91.66 75.0802) (width 0.2) (layer "F.Cu") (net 26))
 (segment (start 78.74 68.58) (end 76.2 68.58) (width 0.2) (layer "F.Cu") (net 26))
 (segment (start 91.66 75.0802) (end 88.2998 71.72) (width 0.2) (layer "F.Cu") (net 26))
 (segment (start 88.2998 71.72) (end 81.28 71.72) (width 0.2) (layer "F.Cu") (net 26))
 (via (at 81.28 71.72) (size 0.6) (drill 0.3) (layers "F.Cu" "B.Cu") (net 26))
 (via (at 78.74 68.58) (size 0.6) (drill 0.3) (layers "F.Cu" "B.Cu") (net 26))
 (segment (start 81.28 71.72) (end 78.74 69.18) (width 0.2) (layer "B.Cu") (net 26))
 (segment (start 78.74 69.18) (end 78.74 68.58) (width 0.2) (layer "B.Cu") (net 26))
 (segment (start 55.88 55.88) (end 56.955 54.805) (width 0.2) (layer "F.Cu") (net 6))
 (segment (start 48.26 58.42) (end 50.8 55.88) (width 0.2) (layer "F.Cu") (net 6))
 (segment (start 50.8 55.88) (end 55.88 55.88) (width 0.2) (layer "F.Cu") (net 6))
 (segment (start 56.955 54.805) (end 91.905 54.805) (width 0.2) (layer "F.Cu") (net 6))
 (segment (start 81.28 93.98) (end 78.96 91.66) (width 0.2) (layer "F.Cu") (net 2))
 (segment (start 52.282132 67.522133) (end 50.8 66.040001) (width 0.2) (layer "F.Cu") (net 2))
 (segment (start 78.96 91.66) (end 76.42 91.66) (width 0.2) (layer "F.Cu") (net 2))
 (segment (start 76.42 91.66) (end 58.42 73.66) (width 0.2) (layer "F.Cu") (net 2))
 (segment (start 50.8 66.040001) (end 50.8 58.42) (width 0.2) (layer "F.Cu") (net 2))
 (via (at 58.42 73.66) (size 0.6) (drill 0.3) (layers "F.Cu" "B.Cu") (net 2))
 (via (at 52.282132 67.522133) (size 0.6) (drill 0.3) (layers "F.Cu" "B.Cu") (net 2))
 (segment (start 52.282133 67.522133) (end 52.282132 67.522133) (width 0.2) (layer "B.Cu") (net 2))
 (segment (start 58.42 73.66) (end 52.282133 67.522133) (width 0.2) (layer "B.Cu") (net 2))
 (segment (start 78.74 63.5) (end 109.22 63.5) (width 0.2) (layer "F.Cu") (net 27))
 (segment (start 109.22 63.5) (end 124.46 78.74) (width 0.2) (layer "F.Cu") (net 27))
 (segment (start 73.66 63.5) (end 68.58 58.42) (width 0.2) (layer "F.Cu") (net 27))
 (via (at 73.66 63.5) (size 0.6) (drill 0.3) (layers "F.Cu" "B.Cu") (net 27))
 (via (at 78.74 63.5) (size 0.6) (drill 0.3) (layers "F.Cu" "B.Cu") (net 27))
 (segment (start 78.74 63.5) (end 73.66 63.5) (width 0.2) (layer "B.Cu") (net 27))
 (segment (start 30.48 93.98) (end 26.79 90.29) (width 0.2) (layer "F.Cu") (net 34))
 (segment (start 26.79 39.25) (end 30.48 35.56) (width 0.2) (layer "F.Cu") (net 34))
 (segment (start 26.79 90.29) (end 26.79 39.25) (width 0.2) (layer "F.Cu") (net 34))
 (segment (start 38.1 78.74) (end 29.09 69.73) (width 0.2) (layer "F.Cu") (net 4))
 (segment (start 29.09 39.49) (end 33.02 35.56) (width 0.2) (layer "F.Cu") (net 4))
 (segment (start 29.09 69.73) (end 29.09 39.49) (width 0.2) (layer "F.Cu") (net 4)))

